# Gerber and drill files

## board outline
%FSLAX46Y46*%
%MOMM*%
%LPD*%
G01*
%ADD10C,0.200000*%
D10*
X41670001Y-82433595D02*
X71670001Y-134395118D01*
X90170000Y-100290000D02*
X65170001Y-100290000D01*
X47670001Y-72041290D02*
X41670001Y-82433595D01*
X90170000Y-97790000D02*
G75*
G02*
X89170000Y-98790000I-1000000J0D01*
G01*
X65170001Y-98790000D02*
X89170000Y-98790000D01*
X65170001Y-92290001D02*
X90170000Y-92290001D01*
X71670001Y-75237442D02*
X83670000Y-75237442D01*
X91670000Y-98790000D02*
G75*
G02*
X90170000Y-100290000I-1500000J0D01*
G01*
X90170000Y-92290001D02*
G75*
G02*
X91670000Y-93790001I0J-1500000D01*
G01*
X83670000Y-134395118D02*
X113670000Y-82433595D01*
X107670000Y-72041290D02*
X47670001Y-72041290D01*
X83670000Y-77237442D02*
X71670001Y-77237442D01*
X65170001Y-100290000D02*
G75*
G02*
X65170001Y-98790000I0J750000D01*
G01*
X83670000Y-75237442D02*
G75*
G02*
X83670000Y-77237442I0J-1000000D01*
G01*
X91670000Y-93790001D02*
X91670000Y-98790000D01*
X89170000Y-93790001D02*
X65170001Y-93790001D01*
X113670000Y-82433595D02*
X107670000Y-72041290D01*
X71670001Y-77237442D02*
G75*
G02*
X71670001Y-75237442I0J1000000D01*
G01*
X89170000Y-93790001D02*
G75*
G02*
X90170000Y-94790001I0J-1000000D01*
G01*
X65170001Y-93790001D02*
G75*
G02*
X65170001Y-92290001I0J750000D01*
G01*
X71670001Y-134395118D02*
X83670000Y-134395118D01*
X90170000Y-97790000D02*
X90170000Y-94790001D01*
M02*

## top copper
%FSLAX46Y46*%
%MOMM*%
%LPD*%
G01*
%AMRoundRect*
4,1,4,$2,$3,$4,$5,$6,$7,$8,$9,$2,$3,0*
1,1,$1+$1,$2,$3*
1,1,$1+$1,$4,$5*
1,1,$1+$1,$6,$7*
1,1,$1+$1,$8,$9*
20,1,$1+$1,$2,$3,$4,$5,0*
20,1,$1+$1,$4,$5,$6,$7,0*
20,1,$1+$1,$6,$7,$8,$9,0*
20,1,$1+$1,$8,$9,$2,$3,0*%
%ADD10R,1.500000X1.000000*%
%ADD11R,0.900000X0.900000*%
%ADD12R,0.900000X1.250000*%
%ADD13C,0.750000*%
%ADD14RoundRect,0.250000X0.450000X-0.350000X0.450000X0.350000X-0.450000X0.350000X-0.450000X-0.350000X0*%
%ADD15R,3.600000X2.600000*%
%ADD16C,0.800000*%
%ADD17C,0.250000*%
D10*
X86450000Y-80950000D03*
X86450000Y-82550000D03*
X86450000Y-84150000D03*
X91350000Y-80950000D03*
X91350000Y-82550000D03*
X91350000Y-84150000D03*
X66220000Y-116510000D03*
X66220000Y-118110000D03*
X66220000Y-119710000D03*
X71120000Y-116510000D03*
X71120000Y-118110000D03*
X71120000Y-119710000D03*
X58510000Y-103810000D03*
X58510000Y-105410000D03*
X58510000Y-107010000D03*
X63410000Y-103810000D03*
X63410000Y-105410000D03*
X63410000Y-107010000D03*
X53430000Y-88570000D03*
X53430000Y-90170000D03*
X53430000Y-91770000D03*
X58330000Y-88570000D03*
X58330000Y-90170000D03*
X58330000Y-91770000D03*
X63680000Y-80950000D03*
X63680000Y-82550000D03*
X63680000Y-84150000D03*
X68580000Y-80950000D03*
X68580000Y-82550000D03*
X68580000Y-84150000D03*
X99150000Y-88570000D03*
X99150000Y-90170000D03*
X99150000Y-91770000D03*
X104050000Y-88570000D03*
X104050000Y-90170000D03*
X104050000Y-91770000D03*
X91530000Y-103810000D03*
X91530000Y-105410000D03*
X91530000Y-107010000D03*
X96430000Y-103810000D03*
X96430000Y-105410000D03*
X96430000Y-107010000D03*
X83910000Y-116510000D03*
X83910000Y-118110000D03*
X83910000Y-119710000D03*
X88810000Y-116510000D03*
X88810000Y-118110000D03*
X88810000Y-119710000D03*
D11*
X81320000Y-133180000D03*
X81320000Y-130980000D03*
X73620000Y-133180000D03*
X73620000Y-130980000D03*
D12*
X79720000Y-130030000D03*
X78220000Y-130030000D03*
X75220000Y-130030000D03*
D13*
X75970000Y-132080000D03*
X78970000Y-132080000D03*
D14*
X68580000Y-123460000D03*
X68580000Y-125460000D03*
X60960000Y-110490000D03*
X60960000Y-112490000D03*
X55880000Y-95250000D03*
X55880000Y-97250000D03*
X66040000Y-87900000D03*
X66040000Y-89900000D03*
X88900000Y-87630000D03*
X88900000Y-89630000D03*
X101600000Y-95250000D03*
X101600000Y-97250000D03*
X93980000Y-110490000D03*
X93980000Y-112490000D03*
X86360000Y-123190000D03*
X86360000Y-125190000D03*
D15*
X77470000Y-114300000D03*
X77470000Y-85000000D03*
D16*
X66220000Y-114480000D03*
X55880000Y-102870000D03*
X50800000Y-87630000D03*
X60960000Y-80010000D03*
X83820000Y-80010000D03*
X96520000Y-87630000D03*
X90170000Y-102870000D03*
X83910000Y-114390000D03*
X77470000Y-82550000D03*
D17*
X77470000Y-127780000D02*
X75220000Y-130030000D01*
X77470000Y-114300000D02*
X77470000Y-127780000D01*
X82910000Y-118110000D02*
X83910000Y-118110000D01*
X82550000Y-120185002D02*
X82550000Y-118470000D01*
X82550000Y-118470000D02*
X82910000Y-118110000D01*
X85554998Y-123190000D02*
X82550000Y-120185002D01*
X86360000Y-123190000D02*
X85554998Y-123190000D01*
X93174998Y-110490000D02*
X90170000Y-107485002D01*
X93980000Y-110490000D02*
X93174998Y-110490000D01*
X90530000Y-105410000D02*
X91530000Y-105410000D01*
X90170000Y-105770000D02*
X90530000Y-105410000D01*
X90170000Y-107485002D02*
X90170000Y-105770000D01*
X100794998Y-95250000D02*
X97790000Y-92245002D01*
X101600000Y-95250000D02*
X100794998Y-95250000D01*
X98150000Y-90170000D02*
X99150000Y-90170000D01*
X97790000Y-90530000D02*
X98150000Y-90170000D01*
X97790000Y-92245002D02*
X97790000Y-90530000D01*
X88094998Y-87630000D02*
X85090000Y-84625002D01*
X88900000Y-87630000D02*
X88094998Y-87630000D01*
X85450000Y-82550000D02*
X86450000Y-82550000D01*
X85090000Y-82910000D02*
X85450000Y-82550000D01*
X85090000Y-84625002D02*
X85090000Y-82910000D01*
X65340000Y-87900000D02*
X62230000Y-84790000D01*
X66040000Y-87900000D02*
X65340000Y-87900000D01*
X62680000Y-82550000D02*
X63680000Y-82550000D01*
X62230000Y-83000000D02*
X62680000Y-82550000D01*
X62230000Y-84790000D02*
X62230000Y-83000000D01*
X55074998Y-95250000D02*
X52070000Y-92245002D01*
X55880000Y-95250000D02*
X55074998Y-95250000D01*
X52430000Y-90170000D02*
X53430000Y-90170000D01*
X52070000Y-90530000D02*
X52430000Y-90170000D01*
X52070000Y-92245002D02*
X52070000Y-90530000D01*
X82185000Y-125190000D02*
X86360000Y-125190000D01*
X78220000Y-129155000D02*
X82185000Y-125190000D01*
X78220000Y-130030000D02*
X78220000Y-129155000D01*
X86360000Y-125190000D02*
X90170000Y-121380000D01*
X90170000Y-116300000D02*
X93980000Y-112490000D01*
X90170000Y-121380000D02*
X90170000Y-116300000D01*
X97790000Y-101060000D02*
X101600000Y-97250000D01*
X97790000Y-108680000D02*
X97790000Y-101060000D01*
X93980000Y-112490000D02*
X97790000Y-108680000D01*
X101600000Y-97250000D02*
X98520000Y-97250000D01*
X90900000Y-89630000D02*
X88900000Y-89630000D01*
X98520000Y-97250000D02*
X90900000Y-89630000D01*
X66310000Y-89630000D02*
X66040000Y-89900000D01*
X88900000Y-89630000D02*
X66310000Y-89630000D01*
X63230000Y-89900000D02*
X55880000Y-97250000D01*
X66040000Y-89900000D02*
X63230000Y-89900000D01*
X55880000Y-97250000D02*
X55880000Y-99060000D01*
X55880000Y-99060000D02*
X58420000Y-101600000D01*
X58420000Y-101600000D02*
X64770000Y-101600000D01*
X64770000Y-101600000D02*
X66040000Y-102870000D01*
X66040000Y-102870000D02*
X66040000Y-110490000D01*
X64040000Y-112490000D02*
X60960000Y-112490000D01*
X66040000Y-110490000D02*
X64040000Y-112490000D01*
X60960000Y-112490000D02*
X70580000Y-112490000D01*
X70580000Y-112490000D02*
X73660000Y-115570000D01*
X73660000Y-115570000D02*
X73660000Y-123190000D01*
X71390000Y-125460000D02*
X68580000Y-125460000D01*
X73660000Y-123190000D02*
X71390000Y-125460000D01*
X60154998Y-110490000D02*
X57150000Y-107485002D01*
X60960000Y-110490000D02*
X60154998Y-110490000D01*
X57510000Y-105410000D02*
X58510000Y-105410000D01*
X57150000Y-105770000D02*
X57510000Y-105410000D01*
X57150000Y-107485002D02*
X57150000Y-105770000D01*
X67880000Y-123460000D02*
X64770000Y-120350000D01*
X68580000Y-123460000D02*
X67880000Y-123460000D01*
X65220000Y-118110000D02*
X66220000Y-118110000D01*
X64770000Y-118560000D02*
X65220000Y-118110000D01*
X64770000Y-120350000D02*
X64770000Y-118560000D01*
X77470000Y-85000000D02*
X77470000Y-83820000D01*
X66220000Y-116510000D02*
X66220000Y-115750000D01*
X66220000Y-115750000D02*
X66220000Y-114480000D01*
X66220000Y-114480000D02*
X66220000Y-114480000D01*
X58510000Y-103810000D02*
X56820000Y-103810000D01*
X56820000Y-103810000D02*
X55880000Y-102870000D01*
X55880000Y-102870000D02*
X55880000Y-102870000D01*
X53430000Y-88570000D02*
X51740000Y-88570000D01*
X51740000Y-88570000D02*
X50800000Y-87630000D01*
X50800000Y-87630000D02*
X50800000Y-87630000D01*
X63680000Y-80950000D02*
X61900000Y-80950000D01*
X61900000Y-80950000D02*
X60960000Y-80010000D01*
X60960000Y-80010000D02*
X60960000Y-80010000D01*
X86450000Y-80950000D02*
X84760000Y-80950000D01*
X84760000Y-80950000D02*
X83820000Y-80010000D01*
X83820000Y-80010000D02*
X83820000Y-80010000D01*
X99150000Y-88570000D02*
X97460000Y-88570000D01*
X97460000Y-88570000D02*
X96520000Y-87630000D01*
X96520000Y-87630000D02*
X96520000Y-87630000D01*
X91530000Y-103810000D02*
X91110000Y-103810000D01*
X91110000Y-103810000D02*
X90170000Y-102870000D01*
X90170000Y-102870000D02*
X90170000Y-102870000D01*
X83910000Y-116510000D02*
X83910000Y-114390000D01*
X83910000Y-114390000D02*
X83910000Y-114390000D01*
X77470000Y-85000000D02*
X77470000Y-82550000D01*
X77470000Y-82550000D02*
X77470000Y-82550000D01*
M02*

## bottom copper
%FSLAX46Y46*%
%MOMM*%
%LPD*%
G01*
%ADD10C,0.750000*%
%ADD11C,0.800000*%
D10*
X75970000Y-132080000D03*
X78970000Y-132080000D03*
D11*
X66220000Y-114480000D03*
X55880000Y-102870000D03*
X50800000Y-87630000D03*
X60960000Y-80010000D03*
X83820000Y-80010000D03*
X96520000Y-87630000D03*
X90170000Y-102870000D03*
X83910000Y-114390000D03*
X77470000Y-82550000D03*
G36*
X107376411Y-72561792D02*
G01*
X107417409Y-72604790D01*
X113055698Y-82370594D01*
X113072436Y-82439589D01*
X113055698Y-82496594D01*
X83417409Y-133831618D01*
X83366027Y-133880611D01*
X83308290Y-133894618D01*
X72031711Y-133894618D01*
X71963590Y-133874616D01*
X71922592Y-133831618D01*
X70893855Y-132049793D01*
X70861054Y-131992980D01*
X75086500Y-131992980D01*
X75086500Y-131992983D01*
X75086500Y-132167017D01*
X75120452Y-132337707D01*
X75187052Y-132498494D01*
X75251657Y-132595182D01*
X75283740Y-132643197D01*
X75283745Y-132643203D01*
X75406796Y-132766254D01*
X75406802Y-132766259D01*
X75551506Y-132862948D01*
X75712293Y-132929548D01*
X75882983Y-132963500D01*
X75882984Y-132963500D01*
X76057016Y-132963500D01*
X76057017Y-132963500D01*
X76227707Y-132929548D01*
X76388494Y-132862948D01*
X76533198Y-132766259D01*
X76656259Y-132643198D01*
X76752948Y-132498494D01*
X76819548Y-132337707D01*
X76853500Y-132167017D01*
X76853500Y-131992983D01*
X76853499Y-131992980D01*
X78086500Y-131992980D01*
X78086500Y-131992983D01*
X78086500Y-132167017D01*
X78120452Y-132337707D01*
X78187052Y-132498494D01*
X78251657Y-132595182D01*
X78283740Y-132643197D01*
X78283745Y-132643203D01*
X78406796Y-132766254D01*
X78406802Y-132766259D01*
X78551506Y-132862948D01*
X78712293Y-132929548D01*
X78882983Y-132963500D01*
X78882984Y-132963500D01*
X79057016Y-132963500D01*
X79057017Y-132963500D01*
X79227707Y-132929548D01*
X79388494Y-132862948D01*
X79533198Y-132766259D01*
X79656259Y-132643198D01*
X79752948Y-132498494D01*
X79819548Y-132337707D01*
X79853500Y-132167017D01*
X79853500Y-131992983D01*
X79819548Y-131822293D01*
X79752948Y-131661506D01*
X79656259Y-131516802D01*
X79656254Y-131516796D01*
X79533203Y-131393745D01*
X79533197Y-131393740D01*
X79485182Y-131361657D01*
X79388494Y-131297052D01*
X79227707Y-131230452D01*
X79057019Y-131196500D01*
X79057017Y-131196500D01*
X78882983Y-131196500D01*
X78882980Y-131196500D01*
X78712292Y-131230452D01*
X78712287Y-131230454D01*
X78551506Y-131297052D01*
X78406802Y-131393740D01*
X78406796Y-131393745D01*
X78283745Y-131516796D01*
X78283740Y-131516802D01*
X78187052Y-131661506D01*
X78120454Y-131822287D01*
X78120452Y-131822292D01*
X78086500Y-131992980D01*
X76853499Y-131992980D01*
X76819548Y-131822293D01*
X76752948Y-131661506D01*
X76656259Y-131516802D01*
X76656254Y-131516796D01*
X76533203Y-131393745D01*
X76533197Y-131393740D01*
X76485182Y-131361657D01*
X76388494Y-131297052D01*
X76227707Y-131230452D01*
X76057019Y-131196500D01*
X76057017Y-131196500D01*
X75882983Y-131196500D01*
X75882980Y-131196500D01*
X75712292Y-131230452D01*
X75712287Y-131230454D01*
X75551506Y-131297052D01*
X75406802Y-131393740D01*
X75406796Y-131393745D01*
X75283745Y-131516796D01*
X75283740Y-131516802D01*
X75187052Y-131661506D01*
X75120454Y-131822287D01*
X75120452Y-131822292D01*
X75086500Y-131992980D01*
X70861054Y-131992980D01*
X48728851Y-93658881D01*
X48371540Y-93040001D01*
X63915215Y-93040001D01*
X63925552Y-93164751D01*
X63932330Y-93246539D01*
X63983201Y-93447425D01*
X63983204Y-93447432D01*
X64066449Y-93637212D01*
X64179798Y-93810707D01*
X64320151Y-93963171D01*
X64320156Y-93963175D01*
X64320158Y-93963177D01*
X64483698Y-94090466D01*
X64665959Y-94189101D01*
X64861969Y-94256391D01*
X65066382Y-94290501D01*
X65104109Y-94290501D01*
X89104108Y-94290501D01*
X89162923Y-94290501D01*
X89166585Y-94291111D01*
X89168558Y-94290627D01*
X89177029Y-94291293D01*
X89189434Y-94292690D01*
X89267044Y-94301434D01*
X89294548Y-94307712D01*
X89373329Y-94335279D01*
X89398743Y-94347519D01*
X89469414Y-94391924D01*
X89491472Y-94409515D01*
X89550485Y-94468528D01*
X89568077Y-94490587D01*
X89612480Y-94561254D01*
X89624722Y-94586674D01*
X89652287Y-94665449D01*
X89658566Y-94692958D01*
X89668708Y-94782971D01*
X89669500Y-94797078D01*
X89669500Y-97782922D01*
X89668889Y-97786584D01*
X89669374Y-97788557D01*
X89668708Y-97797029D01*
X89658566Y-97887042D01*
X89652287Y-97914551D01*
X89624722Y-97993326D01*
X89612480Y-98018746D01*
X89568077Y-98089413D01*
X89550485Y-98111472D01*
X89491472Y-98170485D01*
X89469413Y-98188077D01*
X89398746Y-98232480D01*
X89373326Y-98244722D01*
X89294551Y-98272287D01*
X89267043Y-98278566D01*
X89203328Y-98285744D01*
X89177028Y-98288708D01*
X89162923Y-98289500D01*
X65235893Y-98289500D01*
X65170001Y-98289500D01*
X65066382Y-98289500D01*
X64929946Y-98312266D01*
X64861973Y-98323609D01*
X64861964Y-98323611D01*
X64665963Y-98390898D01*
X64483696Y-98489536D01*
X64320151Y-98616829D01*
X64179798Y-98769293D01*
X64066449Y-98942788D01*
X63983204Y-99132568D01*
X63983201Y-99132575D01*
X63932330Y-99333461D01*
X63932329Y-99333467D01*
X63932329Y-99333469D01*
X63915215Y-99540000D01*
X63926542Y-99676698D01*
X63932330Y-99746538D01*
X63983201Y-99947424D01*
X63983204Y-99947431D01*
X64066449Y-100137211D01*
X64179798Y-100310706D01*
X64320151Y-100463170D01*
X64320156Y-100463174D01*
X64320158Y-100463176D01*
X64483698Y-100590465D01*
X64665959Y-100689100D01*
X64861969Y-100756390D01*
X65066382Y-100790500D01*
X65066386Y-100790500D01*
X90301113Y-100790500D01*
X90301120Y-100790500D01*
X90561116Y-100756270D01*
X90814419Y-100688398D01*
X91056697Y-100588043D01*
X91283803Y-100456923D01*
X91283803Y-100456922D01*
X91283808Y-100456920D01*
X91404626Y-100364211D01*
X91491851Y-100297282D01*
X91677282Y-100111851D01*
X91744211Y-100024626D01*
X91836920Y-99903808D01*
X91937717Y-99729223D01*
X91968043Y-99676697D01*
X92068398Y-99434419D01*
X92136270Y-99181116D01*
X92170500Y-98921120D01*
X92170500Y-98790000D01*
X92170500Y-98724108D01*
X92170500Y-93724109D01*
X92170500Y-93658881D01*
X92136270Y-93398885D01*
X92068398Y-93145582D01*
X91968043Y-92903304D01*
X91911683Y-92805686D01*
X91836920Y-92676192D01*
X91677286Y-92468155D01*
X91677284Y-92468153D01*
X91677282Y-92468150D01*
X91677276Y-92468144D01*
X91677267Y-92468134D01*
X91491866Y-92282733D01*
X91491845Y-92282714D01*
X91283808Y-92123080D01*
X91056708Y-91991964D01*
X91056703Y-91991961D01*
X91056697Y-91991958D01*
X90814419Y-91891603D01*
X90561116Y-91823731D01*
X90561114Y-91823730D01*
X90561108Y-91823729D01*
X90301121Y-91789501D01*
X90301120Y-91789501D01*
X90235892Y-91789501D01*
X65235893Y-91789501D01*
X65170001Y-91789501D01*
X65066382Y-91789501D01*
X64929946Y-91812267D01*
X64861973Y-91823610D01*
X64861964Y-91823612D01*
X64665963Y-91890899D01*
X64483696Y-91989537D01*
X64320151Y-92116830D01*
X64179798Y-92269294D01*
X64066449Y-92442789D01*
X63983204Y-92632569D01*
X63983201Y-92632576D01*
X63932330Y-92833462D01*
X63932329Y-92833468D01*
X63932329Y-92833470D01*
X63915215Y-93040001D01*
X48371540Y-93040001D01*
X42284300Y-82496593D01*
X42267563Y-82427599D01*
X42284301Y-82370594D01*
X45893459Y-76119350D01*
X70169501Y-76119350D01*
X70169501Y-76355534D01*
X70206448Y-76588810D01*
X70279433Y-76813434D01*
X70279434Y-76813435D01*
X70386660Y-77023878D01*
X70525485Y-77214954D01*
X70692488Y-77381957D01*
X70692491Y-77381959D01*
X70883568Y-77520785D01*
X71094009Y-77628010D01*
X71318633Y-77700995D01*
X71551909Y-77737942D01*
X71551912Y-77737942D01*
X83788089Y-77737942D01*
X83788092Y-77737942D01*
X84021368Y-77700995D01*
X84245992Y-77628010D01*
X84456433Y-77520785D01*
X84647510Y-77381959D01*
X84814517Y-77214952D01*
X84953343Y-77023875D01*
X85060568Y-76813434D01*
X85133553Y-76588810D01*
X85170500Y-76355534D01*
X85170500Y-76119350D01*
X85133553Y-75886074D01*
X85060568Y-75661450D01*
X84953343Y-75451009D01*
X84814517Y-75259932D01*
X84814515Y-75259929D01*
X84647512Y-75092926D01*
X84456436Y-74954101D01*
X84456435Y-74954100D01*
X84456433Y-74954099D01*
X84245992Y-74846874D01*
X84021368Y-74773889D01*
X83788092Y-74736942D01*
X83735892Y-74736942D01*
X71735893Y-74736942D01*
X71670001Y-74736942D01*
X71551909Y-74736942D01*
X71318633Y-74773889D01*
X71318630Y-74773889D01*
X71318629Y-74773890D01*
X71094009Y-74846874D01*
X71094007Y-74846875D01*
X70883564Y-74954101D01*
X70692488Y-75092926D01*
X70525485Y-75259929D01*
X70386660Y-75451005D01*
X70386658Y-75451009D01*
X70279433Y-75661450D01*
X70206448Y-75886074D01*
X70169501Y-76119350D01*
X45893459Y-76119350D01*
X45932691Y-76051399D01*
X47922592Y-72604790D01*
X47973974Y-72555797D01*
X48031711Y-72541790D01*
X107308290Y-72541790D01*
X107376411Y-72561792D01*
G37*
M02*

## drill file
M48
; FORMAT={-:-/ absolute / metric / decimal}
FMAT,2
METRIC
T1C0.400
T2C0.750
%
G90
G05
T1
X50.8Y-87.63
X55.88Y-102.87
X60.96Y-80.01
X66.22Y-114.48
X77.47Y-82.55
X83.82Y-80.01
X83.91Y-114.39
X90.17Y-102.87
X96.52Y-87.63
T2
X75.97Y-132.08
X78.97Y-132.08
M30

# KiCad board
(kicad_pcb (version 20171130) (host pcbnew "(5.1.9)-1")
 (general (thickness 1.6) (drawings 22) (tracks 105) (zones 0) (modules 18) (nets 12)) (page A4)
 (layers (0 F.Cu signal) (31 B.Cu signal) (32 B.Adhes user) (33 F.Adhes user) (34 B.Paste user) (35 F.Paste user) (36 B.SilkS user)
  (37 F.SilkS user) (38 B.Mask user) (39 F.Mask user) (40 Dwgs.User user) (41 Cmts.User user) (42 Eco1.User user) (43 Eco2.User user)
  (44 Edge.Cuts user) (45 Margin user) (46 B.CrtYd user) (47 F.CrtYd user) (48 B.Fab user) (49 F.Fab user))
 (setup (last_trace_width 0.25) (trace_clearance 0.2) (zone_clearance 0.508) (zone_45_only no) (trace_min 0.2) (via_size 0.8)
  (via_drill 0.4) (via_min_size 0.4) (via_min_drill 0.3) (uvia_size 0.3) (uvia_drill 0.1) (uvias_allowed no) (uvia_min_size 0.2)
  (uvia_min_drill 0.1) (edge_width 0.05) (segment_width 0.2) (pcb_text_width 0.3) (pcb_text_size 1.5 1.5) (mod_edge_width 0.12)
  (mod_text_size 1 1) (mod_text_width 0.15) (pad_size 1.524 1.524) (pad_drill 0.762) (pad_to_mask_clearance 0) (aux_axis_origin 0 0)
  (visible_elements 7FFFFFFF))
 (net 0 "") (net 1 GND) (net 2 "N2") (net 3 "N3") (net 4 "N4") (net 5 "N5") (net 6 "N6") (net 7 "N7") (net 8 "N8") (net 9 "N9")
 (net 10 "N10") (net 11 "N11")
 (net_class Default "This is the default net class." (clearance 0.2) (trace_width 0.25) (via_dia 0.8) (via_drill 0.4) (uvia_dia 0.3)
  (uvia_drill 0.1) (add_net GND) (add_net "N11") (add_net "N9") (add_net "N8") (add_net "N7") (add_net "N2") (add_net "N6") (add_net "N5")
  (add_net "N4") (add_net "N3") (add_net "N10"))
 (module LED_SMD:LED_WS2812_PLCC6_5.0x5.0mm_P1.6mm (layer F.Cu) (at 88.9 82.55)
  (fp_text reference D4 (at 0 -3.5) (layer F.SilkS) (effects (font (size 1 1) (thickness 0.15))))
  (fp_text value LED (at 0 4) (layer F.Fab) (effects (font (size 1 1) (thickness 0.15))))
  (pad 1 smd rect (at -2.45 -1.6) (size 1.5 1) (layers F.Cu F.Paste F.Mask) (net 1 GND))
  (pad 2 smd rect (at -2.45 0) (size 1.5 1) (layers F.Cu F.Paste F.Mask) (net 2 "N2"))
  (pad 3 smd rect (at -2.45 1.6) (size 1.5 1) (layers F.Cu F.Paste F.Mask))
  (pad 6 smd rect (at 2.45 -1.6) (size 1.5 1) (layers F.Cu F.Paste F.Mask))
  (pad 5 smd rect (at 2.45 0) (size 1.5 1) (layers F.Cu F.Paste F.Mask))
  (pad 4 smd rect (at 2.45 1.6) (size 1.5 1) (layers F.Cu F.Paste F.Mask)))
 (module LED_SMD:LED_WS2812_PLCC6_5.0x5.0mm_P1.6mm (layer F.Cu) (at 68.67 118.11)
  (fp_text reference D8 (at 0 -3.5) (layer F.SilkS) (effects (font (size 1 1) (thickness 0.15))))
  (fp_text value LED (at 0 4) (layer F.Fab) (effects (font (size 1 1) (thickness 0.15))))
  (pad 1 smd rect (at -2.45 -1.6) (size 1.5 1) (layers F.Cu F.Paste F.Mask) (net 1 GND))
  (pad 2 smd rect (at -2.45 0) (size 1.5 1) (layers F.Cu F.Paste F.Mask) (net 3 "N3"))
  (pad 3 smd rect (at -2.45 1.6) (size 1.5 1) (layers F.Cu F.Paste F.Mask))
  (pad 6 smd rect (at 2.45 -1.6) (size 1.5 1) (layers F.Cu F.Paste F.Mask))
  (pad 5 smd rect (at 2.45 0) (size 1.5 1) (layers F.Cu F.Paste F.Mask))
  (pad 4 smd rect (at 2.45 1.6) (size 1.5 1) (layers F.Cu F.Paste F.Mask)))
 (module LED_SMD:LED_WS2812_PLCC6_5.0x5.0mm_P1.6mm (layer F.Cu) (at 60.96 105.41)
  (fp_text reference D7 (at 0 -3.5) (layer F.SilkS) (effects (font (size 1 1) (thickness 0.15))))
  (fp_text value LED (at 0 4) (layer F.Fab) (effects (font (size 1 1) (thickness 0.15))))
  (pad 1 smd rect (at -2.45 -1.6) (size 1.5 1) (layers F.Cu F.Paste F.Mask) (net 1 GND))
  (pad 2 smd rect (at -2.45 0) (size 1.5 1) (layers F.Cu F.Paste F.Mask) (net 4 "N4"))
  (pad 3 smd rect (at -2.45 1.6) (size 1.5 1) (layers F.Cu F.Paste F.Mask))
  (pad 6 smd rect (at 2.45 -1.6) (size 1.5 1) (layers F.Cu F.Paste F.Mask))
  (pad 5 smd rect (at 2.45 0) (size 1.5 1) (layers F.Cu F.Paste F.Mask))
  (pad 4 smd rect (at 2.45 1.6) (size 1.5 1) (layers F.Cu F.Paste F.Mask)))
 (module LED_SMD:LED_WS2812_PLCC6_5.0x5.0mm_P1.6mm (layer F.Cu) (at 55.88 90.17)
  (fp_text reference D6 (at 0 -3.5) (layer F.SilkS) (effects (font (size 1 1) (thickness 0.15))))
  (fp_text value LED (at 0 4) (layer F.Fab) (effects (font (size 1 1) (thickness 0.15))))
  (pad 1 smd rect (at -2.45 -1.6) (size 1.5 1) (layers F.Cu F.Paste F.Mask) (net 1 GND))
  (pad 2 smd rect (at -2.45 0) (size 1.5 1) (layers F.Cu F.Paste F.Mask) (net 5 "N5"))
  (pad 3 smd rect (at -2.45 1.6) (size 1.5 1) (layers F.Cu F.Paste F.Mask))
  (pad 6 smd rect (at 2.45 -1.6) (size 1.5 1) (layers F.Cu F.Paste F.Mask))
  (pad 5 smd rect (at 2.45 0) (size 1.5 1) (layers F.Cu F.Paste F.Mask))
  (pad 4 smd rect (at 2.45 1.6) (size 1.5 1) (layers F.Cu F.Paste F.Mask)))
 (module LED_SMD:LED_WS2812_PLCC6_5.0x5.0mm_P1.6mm (layer F.Cu) (at 66.13 82.55)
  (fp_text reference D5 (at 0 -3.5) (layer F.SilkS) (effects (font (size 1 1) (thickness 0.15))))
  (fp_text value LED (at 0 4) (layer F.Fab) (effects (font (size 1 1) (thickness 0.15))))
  (pad 1 smd rect (at -2.45 -1.6) (size 1.5 1) (layers F.Cu F.Paste F.Mask) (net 1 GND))
  (pad 2 smd rect (at -2.45 0) (size 1.5 1) (layers F.Cu F.Paste F.Mask) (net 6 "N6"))
  (pad 3 smd rect (at -2.45 1.6) (size 1.5 1) (layers F.Cu F.Paste F.Mask))
  (pad 6 smd rect (at 2.45 -1.6) (size 1.5 1) (layers F.Cu F.Paste F.Mask))
  (pad 5 smd rect (at 2.45 0) (size 1.5 1) (layers F.Cu F.Paste F.Mask))
  (pad 4 smd rect (at 2.45 1.6) (size 1.5 1) (layers F.Cu F.Paste F.Mask)))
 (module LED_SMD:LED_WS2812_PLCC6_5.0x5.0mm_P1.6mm (layer F.Cu) (at 101.6 90.17)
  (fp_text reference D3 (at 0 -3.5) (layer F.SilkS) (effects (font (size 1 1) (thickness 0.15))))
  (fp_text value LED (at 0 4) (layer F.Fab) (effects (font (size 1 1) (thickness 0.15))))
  (pad 1 smd rect (at -2.45 -1.6) (size 1.5 1) (layers F.Cu F.Paste F.Mask) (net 1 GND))
  (pad 2 smd rect (at -2.45 0) (size 1.5 1) (layers F.Cu F.Paste F.Mask) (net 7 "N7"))
  (pad 3 smd rect (at -2.45 1.6) (size 1.5 1) (layers F.Cu F.Paste F.Mask))
  (pad 6 smd rect (at 2.45 -1.6) (size 1.5 1) (layers F.Cu F.Paste F.Mask))
  (pad 5 smd rect (at 2.45 0) (size 1.5 1) (layers F.Cu F.Paste F.Mask))
  (pad 4 smd rect (at 2.45 1.6) (size 1.5 1) (layers F.Cu F.Paste F.Mask)))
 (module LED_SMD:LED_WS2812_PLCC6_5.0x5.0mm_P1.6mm (layer F.Cu) (at 93.98 105.41)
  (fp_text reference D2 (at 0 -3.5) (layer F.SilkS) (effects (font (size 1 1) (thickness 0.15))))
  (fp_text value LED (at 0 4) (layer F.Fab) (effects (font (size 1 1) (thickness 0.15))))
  (pad 1 smd rect (at -2.45 -1.6) (size 1.5 1) (layers F.Cu F.Paste F.Mask) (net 1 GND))
  (pad 2 smd rect (at -2.45 0) (size 1.5 1) (layers F.Cu F.Paste F.Mask) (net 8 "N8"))
  (pad 3 smd rect (at -2.45 1.6) (size 1.5 1) (layers F.Cu F.Paste F.Mask))
  (pad 6 smd rect (at 2.45 -1.6) (size 1.5 1) (layers F.Cu F.Paste F.Mask))
  (pad 5 smd rect (at 2.45 0) (size 1.5 1) (layers F.Cu F.Paste F.Mask))
  (pad 4 smd rect (at 2.45 1.6) (size 1.5 1) (layers F.Cu F.Paste F.Mask)))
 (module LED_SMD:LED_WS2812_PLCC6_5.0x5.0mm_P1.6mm (layer F.Cu) (at 86.36 118.11)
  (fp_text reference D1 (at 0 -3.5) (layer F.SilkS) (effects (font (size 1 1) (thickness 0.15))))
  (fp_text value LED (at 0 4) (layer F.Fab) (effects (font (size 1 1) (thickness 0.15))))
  (pad 1 smd rect (at -2.45 -1.6) (size 1.5 1) (layers F.Cu F.Paste F.Mask) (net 1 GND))
  (pad 2 smd rect (at -2.45 0) (size 1.5 1) (layers F.Cu F.Paste F.Mask) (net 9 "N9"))
  (pad 3 smd rect (at -2.45 1.6) (size 1.5 1) (layers F.Cu F.Paste F.Mask))
  (pad 6 smd rect (at 2.45 -1.6) (size 1.5 1) (layers F.Cu F.Paste F.Mask))
  (pad 5 smd rect (at 2.45 0) (size 1.5 1) (layers F.Cu F.Paste F.Mask))
  (pad 4 smd rect (at 2.45 1.6) (size 1.5 1) (layers F.Cu F.Paste F.Mask)))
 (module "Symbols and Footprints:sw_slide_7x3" (layer F.Cu) (at 77.47 132.08)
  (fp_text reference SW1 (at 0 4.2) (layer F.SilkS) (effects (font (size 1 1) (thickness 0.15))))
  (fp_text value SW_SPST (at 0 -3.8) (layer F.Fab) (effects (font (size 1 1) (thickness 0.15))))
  (pad 4 smd rect (at 3.85 1.1) (size 0.9 0.9) (layers F.Cu F.Paste F.Mask))
  (pad 4 smd rect (at 3.85 -1.1) (size 0.9 0.9) (layers F.Cu F.Paste F.Mask))
  (pad 4 smd rect (at -3.85 1.1) (size 0.9 0.9) (layers F.Cu F.Paste F.Mask))
  (pad 4 smd rect (at -3.85 -1.1) (size 0.9 0.9) (layers F.Cu F.Paste F.Mask))
  (pad 3 smd rect (at 2.25 -2.05) (size 0.9 1.25) (layers F.Cu F.Paste F.Mask))
  (pad 2 smd rect (at 0.75 -2.05) (size 0.9 1.25) (layers F.Cu F.Paste F.Mask) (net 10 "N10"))
  (pad 1 smd rect (at -2.25 -2.05) (size 0.9 1.25) (layers F.Cu F.Paste F.Mask) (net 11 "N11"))
  (pad ~ thru_hole circle (at -1.5 0) (size 0.75 0.75) (drill 0.75) (layers *.Cu *.Mask))
  (pad ~ thru_hole circle (at 1.5 0) (size 0.75 0.75) (drill 0.75) (layers *.Cu *.Mask)))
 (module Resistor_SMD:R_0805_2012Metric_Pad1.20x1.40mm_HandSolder (layer F.Cu) (at 68.58 124.46 90)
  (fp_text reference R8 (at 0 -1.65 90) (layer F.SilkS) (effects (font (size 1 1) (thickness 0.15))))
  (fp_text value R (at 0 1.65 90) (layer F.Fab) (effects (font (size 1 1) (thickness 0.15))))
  (pad 2 smd roundrect (at 1 0 90) (size 1.2 1.4) (layers F.Cu F.Paste F.Mask) (roundrect_rratio 0.208333) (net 3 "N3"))
  (pad 1 smd roundrect (at -1 0 90) (size 1.2 1.4) (layers F.Cu F.Paste F.Mask) (roundrect_rratio 0.208333) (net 10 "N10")))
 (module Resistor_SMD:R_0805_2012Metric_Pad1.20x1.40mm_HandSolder (layer F.Cu) (at 60.96 111.49 90)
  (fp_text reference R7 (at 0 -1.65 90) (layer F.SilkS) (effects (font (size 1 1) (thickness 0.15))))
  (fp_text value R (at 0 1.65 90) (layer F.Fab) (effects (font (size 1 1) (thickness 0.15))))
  (pad 2 smd roundrect (at 1 0 90) (size 1.2 1.4) (layers F.Cu F.Paste F.Mask) (roundrect_rratio 0.208333) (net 4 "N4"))
  (pad 1 smd roundrect (at -1 0 90) (size 1.2 1.4) (layers F.Cu F.Paste F.Mask) (roundrect_rratio 0.208333) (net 10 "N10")))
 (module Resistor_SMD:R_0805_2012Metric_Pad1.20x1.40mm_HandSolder (layer F.Cu) (at 55.88 96.25 90)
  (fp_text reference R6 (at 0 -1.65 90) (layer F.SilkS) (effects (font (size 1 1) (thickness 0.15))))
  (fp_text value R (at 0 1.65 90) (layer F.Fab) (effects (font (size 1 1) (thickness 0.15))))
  (pad 2 smd roundrect (at 1 0 90) (size 1.2 1.4) (layers F.Cu F.Paste F.Mask) (roundrect_rratio 0.208333) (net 5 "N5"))
  (pad 1 smd roundrect (at -1 0 90) (size 1.2 1.4) (layers F.Cu F.Paste F.Mask) (roundrect_rratio 0.208333) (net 10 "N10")))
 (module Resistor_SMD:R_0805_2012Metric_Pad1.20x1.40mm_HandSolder (layer F.Cu) (at 66.04 88.9 90)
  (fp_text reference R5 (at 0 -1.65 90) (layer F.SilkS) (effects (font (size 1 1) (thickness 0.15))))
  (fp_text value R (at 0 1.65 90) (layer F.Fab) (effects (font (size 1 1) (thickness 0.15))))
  (pad 2 smd roundrect (at 1 0 90) (size 1.2 1.4) (layers F.Cu F.Paste F.Mask) (roundrect_rratio 0.208333) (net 6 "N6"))
  (pad 1 smd roundrect (at -1 0 90) (size 1.2 1.4) (layers F.Cu F.Paste F.Mask) (roundrect_rratio 0.208333) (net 10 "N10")))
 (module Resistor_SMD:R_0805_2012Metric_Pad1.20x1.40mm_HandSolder (layer F.Cu) (at 88.9 88.63 90)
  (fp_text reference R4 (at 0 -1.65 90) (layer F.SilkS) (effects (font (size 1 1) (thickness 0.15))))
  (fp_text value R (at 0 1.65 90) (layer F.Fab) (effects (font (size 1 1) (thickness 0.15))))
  (pad 2 smd roundrect (at 1 0 90) (size 1.2 1.4) (layers F.Cu F.Paste F.Mask) (roundrect_rratio 0.208333) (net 2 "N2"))
  (pad 1 smd roundrect (at -1 0 90) (size 1.2 1.4) (layers F.Cu F.Paste F.Mask) (roundrect_rratio 0.208333) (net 10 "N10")))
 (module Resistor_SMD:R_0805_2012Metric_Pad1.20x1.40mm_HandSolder (layer F.Cu) (at 101.6 96.25 90)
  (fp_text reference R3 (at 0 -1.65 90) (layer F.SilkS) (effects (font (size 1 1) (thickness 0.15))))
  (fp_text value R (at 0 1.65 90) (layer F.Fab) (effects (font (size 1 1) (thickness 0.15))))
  (pad 2 smd roundrect (at 1 0 90) (size 1.2 1.4) (layers F.Cu F.Paste F.Mask) (roundrect_rratio 0.208333) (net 7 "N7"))
  (pad 1 smd roundrect (at -1 0 90) (size 1.2 1.4) (layers F.Cu F.Paste F.Mask) (roundrect_rratio 0.208333) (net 10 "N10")))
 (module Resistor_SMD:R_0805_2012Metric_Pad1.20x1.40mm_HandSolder (layer F.Cu) (at 93.98 111.49 90)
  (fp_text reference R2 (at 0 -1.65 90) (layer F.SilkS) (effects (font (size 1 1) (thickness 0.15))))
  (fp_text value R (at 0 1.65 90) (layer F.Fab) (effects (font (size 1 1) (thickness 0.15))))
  (pad 2 smd roundrect (at 1 0 90) (size 1.2 1.4) (layers F.Cu F.Paste F.Mask) (roundrect_rratio 0.208333) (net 8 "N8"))
  (pad 1 smd roundrect (at -1 0 90) (size 1.2 1.4) (layers F.Cu F.Paste F.Mask) (roundrect_rratio 0.208333) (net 10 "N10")))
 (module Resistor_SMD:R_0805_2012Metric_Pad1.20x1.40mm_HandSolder (layer F.Cu) (at 86.36 124.19 90)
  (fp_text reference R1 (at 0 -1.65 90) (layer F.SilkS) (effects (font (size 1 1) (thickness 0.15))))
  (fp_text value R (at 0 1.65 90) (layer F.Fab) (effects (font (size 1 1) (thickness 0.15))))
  (pad 2 smd roundrect (at 1 0 90) (size 1.2 1.4) (layers F.Cu F.Paste F.Mask) (roundrect_rratio 0.208333) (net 9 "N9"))
  (pad 1 smd roundrect (at -1 0 90) (size 1.2 1.4) (layers F.Cu F.Paste F.Mask) (roundrect_rratio 0.208333) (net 10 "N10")))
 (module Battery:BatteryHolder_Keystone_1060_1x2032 (layer F.Cu) (at 77.47 99.65 90)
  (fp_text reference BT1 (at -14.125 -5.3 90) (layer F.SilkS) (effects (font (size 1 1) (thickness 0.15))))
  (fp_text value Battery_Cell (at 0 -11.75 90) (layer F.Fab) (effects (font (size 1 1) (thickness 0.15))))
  (pad 1 smd rect (at -14.65 0 270) (size 2.6 3.6) (layers F.Cu F.Paste F.Mask) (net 11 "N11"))
  (pad 2 smd rect (at 14.65 0 270) (size 2.6 3.6) (layers F.Cu F.Paste F.Mask) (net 1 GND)))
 (gr_line (start 41.670001 82.433595) (end 71.670001 134.395118) (layer Edge.Cuts) (width 0.2))
 (gr_line (start 90.17 100.29) (end 65.170001 100.29) (layer Edge.Cuts) (width 0.2))
 (gr_line (start 47.670001 72.04129) (end 41.670001 82.433595) (layer Edge.Cuts) (width 0.2))
 (gr_arc (start 89.17 97.79) (end 89.17 98.79) (angle -90) (layer Edge.Cuts) (width 0.2))
 (gr_line (start 65.170001 98.79) (end 89.17 98.79) (layer Edge.Cuts) (width 0.2))
 (gr_line (start 65.170001 92.290001) (end 90.17 92.290001) (layer Edge.Cuts) (width 0.2))
 (gr_line (start 71.670001 75.237442) (end 83.67 75.237442) (layer Edge.Cuts) (width 0.2))
 (gr_arc (start 90.17 98.79) (end 90.17 100.29) (angle -90) (layer Edge.Cuts) (width 0.2))
 (gr_arc (start 90.17 93.790001) (end 91.67 93.790001) (angle -90) (layer Edge.Cuts) (width 0.2))
 (gr_line (start 83.67 134.395118) (end 113.67 82.433595) (layer Edge.Cuts) (width 0.2))
 (gr_line (start 107.67 72.04129) (end 47.670001 72.04129) (layer Edge.Cuts) (width 0.2))
 (gr_line (start 83.67 77.237442) (end 71.670001 77.237442) (layer Edge.Cuts) (width 0.2))
 (gr_arc (start 65.170001 99.54) (end 65.170001 98.79) (angle -180) (layer Edge.Cuts) (width 0.2))
 (gr_arc (start 83.67 76.237442) (end 83.67 77.237442) (angle -180) (layer Edge.Cuts) (width 0.2))
 (gr_line (start 91.67 93.790001) (end 91.67 98.79) (layer Edge.Cuts) (width 0.2))
 (gr_line (start 89.17 93.790001) (end 65.170001 93.790001) (layer Edge.Cuts) (width 0.2))
 (gr_line (start 113.67 82.433595) (end 107.67 72.04129) (layer Edge.Cuts) (width 0.2))
 (gr_arc (start 71.670001 76.237442) (end 71.670001 75.237442) (angle -180) (layer Edge.Cuts) (width 0.2))
 (gr_arc (start 89.17 94.790001) (end 90.17 94.790001) (angle -90) (layer Edge.Cuts) (width 0.2))
 (gr_arc (start 65.170001 93.040001) (end 65.170001 92.290001) (angle -180) (layer Edge.Cuts) (width 0.2))
 (gr_line (start 71.670001 134.395118) (end 83.67 134.395118) (layer Edge.Cuts) (width 0.2))
 (gr_line (start 90.17 97.79) (end 90.17 94.790001) (layer Edge.Cuts) (width 0.2))
 (segment (start 77.47 127.78) (end 75.22 130.03) (width 0.25) (layer F.Cu) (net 11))
 (segment (start 77.47 114.3) (end 77.47 127.78) (width 0.25) (layer F.Cu) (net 11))
 (segment (start 82.91 118.11) (end 83.91 118.11) (width 0.25) (layer F.Cu) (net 9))
 (segment (start 82.55 120.185002) (end 82.55 118.47) (width 0.25) (layer F.Cu) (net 9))
 (segment (start 82.55 118.47) (end 82.91 118.11) (width 0.25) (layer F.Cu) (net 9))
 (segment (start 85.554998 123.19) (end 82.55 120.185002) (width 0.25) (layer F.Cu) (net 9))
 (segment (start 86.36 123.19) (end 85.554998 123.19) (width 0.25) (layer F.Cu) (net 9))
 (segment (start 93.174998 110.49) (end 90.17 107.485002) (width 0.25) (layer F.Cu) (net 8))
 (segment (start 93.98 110.49) (end 93.174998 110.49) (width 0.25) (layer F.Cu) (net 8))
 (segment (start 90.53 105.41) (end 91.53 105.41) (width 0.25) (layer F.Cu) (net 8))
 (segment (start 90.17 105.77) (end 90.53 105.41) (width 0.25) (layer F.Cu) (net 8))
 (segment (start 90.17 107.485002) (end 90.17 105.77) (width 0.25) (layer F.Cu) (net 8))
 (segment (start 100.794998 95.25) (end 97.79 92.245002) (width 0.25) (layer F.Cu) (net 7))
 (segment (start 101.6 95.25) (end 100.794998 95.25) (width 0.25) (layer F.Cu) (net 7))
 (segment (start 98.15 90.17) (end 99.15 90.17) (width 0.25) (layer F.Cu) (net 7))
 (segment (start 97.79 90.53) (end 98.15 90.17) (width 0.25) (layer F.Cu) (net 7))
 (segment (start 97.79 92.245002) (end 97.79 90.53) (width 0.25) (layer F.Cu) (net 7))
 (segment (start 88.094998 87.63) (end 85.09 84.625002) (width 0.25) (layer F.Cu) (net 2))
 (segment (start 88.9 87.63) (end 88.094998 87.63) (width 0.25) (layer F.Cu) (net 2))
 (segment (start 85.45 82.55) (end 86.45 82.55) (width 0.25) (layer F.Cu) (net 2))
 (segment (start 85.09 82.91) (end 85.45 82.55) (width 0.25) (layer F.Cu) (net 2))
 (segment (start 85.09 84.625002) (end 85.09 82.91) (width 0.25) (layer F.Cu) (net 2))
 (segment (start 65.34 87.9) (end 62.23 84.79) (width 0.25) (layer F.Cu) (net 6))
 (segment (start 66.04 87.9) (end 65.34 87.9) (width 0.25) (layer F.Cu) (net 6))
 (segment (start 62.68 82.55) (end 63.68 82.55) (width 0.25) (layer F.Cu) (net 6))
 (segment (start 62.23 83) (end 62.68 82.55) (width 0.25) (layer F.Cu) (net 6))
 (segment (start 62.23 84.79) (end 62.23 83) (width 0.25) (layer F.Cu) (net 6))
 (segment (start 55.074998 95.25) (end 52.07 92.245002) (width 0.25) (layer F.Cu) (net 5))
 (segment (start 55.88 95.25) (end 55.074998 95.25) (width 0.25) (layer F.Cu) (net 5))
 (segment (start 52.43 90.17) (end 53.43 90.17) (width 0.25) (layer F.Cu) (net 5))
 (segment (start 52.07 90.53) (end 52.43 90.17) (width 0.25) (layer F.Cu) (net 5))
 (segment (start 52.07 92.245002) (end 52.07 90.53) (width 0.25) (layer F.Cu) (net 5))
 (segment (start 82.185 125.19) (end 86.36 125.19) (width 0.25) (layer F.Cu) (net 10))
 (segment (start 78.22 129.155) (end 82.185 125.19) (width 0.25) (layer F.Cu) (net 10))
 (segment (start 78.22 130.03) (end 78.22 129.155) (width 0.25) (layer F.Cu) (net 10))
 (segment (start 86.36 125.19) (end 90.17 121.38) (width 0.25) (layer F.Cu) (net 10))
 (segment (start 90.17 116.3) (end 93.98 112.49) (width 0.25) (layer F.Cu) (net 10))
 (segment (start 90.17 121.38) (end 90.17 116.3) (width 0.25) (layer F.Cu) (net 10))
 (segment (start 97.79 101.06) (end 101.6 97.25) (width 0.25) (layer F.Cu) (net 10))
 (segment (start 97.79 108.68) (end 97.79 101.06) (width 0.25) (layer F.Cu) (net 10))
 (segment (start 93.98 112.49) (end 97.79 108.68) (width 0.25) (layer F.Cu) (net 10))
 (segment (start 101.6 97.25) (end 98.52 97.25) (width 0.25) (layer F.Cu) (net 10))
 (segment (start 90.9 89.63) (end 88.9 89.63) (width 0.25) (layer F.Cu) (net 10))
 (segment (start 98.52 97.25) (end 90.9 89.63) (width 0.25) (layer F.Cu) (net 10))
 (segment (start 66.31 89.63) (end 66.04 89.9) (width 0.25) (layer F.Cu) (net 10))
 (segment (start 88.9 89.63) (end 66.31 89.63) (width 0.25) (layer F.Cu) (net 10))
 (segment (start 63.23 89.9) (end 55.88 97.25) (width 0.25) (layer F.Cu) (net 10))
 (segment (start 66.04 89.9) (end 63.23 89.9) (width 0.25) (layer F.Cu) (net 10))
 (segment (start 55.88 97.25) (end 55.88 99.06) (width 0.25) (layer F.Cu) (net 10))
 (segment (start 55.88 99.06) (end 58.42 101.6) (width 0.25) (layer F.Cu) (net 10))
 (segment (start 58.42 101.6) (end 64.77 101.6) (width 0.25) (layer F.Cu) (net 10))
 (segment (start 64.77 101.6) (end 66.04 102.87) (width 0.25) (layer F.Cu) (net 10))
 (segment (start 66.04 102.87) (end 66.04 110.49) (width 0.25) (layer F.Cu) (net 10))
 (segment (start 64.04 112.49) (end 60.96 112.49) (width 0.25) (layer F.Cu) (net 10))
 (segment (start 66.04 110.49) (end 64.04 112.49) (width 0.25) (layer F.Cu) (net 10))
 (segment (start 60.96 112.49) (end 70.58 112.49) (width 0.25) (layer F.Cu) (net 10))
 (segment (start 70.58 112.49) (end 73.66 115.57) (width 0.25) (layer F.Cu) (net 10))
 (segment (start 73.66 115.57) (end 73.66 123.19) (width 0.25) (layer F.Cu) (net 10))
 (segment (start 71.39 125.46) (end 68.58 125.46) (width 0.25) (layer F.Cu) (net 10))
 (segment (start 73.66 123.19) (end 71.39 125.46) (width 0.25) (layer F.Cu) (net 10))
 (segment (start 60.154998 110.49) (end 57.15 107.485002) (width 0.25) (layer F.Cu) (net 4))
 (segment (start 60.96 110.49) (end 60.154998 110.49) (width 0.25) (layer F.Cu) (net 4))
 (segment (start 57.51 105.41) (end 58.51 105.41) (width 0.25) (layer F.Cu) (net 4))
 (segment (start 57.15 105.77) (end 57.51 105.41) (width 0.25) (layer F.Cu) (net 4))
 (segment (start 57.15 107.485002) (end 57.15 105.77) (width 0.25) (layer F.Cu) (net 4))
 (segment (start 67.88 123.46) (end 64.77 120.35) (width 0.25) (layer F.Cu) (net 3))
 (segment (start 68.58 123.46) (end 67.88 123.46) (width 0.25) (layer F.Cu) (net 3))
 (segment (start 65.22 118.11) (end 66.22 118.11) (width 0.25) (layer F.Cu) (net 3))
 (segment (start 64.77 118.56) (end 65.22 118.11) (width 0.25) (layer F.Cu) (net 3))
 (segment (start 64.77 120.35) (end 64.77 118.56) (width 0.25) (layer F.Cu) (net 3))
 (segment (start 77.47 85) (end 77.47 83.82) (width 0.25) (layer F.Cu) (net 1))
 (segment (start 66.22 116.51) (end 66.22 115.75) (width 0.25) (layer F.Cu) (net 1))
 (segment (start 66.22 115.75) (end 66.22 114.48) (width 0.25) (layer F.Cu) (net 1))
 (segment (start 66.22 114.48) (end 66.22 114.48) (width 0.25) (layer F.Cu) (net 1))
 (via (at 66.22 114.48) (size 0.8) (drill 0.4) (layers F.Cu B.Cu) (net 1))
 (segment (start 58.51 103.81) (end 56.82 103.81) (width 0.25) (layer F.Cu) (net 1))
 (segment (start 56.82 103.81) (end 55.88 102.87) (width 0.25) (layer F.Cu) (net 1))
 (segment (start 55.88 102.87) (end 55.88 102.87) (width 0.25) (layer F.Cu) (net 1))
 (via (at 55.88 102.87) (size 0.8) (drill 0.4) (layers F.Cu B.Cu) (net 1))
 (segment (start 53.43 88.57) (end 51.74 88.57) (width 0.25) (layer F.Cu) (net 1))
 (segment (start 51.74 88.57) (end 50.8 87.63) (width 0.25) (layer F.Cu) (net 1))
 (segment (start 50.8 87.63) (end 50.8 87.63) (width 0.25) (layer F.Cu) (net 1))
 (via (at 50.8 87.63) (size 0.8) (drill 0.4) (layers F.Cu B.Cu) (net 1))
 (segment (start 63.68 80.95) (end 61.9 80.95) (width 0.25) (layer F.Cu) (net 1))
 (segment (start 61.9 80.95) (end 60.96 80.01) (width 0.25) (layer F.Cu) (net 1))
 (segment (start 60.96 80.01) (end 60.96 80.01) (width 0.25) (layer F.Cu) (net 1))
 (via (at 60.96 80.01) (size 0.8) (drill 0.4) (layers F.Cu B.Cu) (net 1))
 (segment (start 86.45 80.95) (end 84.76 80.95) (width 0.25) (layer F.Cu) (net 1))
 (segment (start 84.76 80.95) (end 83.82 80.01) (width 0.25) (layer F.Cu) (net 1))
 (segment (start 83.82 80.01) (end 83.82 80.01) (width 0.25) (layer F.Cu) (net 1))
 (via (at 83.82 80.01) (size 0.8) (drill 0.4) (layers F.Cu B.Cu) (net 1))
 (segment (start 99.15 88.57) (end 97.46 88.57) (width 0.25) (layer F.Cu) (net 1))
 (segment (start 97.46 88.57) (end 96.52 87.63) (width 0.25) (layer F.Cu) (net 1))
 (segment (start 96.52 87.63) (end 96.52 87.63) (width 0.25) (layer F.Cu) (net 1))
 (via (at 96.52 87.63) (size 0.8) (drill 0.4) (layers F.Cu B.Cu) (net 1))
 (segment (start 91.53 103.81) (end 91.11 103.81) (width 0.25) (layer F.Cu) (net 1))
 (segment (start 91.11 103.81) (end 90.17 102.87) (width 0.25) (layer F.Cu) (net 1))
 (segment (start 90.17 102.87) (end 90.17 102.87) (width 0.25) (layer F.Cu) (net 1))
 (via (at 90.17 102.87) (size 0.8) (drill 0.4) (layers F.Cu B.Cu) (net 1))
 (segment (start 83.91 116.51) (end 83.91 114.39) (width 0.25) (layer F.Cu) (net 1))
 (segment (start 83.91 114.39) (end 83.91 114.39) (width 0.25) (layer F.Cu) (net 1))
 (via (at 83.91 114.39) (size 0.8) (drill 0.4) (layers F.Cu B.Cu) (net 1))
 (segment (start 77.47 85) (end 77.47 82.55) (width 0.25) (layer F.Cu) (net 1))
 (segment (start 77.47 82.55) (end 77.47 82.55) (width 0.25) (layer F.Cu) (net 1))
 (via (at 77.47 82.55) (size 0.8) (drill 0.4) (layers F.Cu B.Cu) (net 1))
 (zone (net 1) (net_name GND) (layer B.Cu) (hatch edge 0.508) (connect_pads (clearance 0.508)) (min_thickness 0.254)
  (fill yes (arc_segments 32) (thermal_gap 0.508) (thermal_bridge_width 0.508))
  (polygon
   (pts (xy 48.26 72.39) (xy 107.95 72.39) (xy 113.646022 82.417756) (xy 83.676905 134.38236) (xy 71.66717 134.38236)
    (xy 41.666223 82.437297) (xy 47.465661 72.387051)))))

